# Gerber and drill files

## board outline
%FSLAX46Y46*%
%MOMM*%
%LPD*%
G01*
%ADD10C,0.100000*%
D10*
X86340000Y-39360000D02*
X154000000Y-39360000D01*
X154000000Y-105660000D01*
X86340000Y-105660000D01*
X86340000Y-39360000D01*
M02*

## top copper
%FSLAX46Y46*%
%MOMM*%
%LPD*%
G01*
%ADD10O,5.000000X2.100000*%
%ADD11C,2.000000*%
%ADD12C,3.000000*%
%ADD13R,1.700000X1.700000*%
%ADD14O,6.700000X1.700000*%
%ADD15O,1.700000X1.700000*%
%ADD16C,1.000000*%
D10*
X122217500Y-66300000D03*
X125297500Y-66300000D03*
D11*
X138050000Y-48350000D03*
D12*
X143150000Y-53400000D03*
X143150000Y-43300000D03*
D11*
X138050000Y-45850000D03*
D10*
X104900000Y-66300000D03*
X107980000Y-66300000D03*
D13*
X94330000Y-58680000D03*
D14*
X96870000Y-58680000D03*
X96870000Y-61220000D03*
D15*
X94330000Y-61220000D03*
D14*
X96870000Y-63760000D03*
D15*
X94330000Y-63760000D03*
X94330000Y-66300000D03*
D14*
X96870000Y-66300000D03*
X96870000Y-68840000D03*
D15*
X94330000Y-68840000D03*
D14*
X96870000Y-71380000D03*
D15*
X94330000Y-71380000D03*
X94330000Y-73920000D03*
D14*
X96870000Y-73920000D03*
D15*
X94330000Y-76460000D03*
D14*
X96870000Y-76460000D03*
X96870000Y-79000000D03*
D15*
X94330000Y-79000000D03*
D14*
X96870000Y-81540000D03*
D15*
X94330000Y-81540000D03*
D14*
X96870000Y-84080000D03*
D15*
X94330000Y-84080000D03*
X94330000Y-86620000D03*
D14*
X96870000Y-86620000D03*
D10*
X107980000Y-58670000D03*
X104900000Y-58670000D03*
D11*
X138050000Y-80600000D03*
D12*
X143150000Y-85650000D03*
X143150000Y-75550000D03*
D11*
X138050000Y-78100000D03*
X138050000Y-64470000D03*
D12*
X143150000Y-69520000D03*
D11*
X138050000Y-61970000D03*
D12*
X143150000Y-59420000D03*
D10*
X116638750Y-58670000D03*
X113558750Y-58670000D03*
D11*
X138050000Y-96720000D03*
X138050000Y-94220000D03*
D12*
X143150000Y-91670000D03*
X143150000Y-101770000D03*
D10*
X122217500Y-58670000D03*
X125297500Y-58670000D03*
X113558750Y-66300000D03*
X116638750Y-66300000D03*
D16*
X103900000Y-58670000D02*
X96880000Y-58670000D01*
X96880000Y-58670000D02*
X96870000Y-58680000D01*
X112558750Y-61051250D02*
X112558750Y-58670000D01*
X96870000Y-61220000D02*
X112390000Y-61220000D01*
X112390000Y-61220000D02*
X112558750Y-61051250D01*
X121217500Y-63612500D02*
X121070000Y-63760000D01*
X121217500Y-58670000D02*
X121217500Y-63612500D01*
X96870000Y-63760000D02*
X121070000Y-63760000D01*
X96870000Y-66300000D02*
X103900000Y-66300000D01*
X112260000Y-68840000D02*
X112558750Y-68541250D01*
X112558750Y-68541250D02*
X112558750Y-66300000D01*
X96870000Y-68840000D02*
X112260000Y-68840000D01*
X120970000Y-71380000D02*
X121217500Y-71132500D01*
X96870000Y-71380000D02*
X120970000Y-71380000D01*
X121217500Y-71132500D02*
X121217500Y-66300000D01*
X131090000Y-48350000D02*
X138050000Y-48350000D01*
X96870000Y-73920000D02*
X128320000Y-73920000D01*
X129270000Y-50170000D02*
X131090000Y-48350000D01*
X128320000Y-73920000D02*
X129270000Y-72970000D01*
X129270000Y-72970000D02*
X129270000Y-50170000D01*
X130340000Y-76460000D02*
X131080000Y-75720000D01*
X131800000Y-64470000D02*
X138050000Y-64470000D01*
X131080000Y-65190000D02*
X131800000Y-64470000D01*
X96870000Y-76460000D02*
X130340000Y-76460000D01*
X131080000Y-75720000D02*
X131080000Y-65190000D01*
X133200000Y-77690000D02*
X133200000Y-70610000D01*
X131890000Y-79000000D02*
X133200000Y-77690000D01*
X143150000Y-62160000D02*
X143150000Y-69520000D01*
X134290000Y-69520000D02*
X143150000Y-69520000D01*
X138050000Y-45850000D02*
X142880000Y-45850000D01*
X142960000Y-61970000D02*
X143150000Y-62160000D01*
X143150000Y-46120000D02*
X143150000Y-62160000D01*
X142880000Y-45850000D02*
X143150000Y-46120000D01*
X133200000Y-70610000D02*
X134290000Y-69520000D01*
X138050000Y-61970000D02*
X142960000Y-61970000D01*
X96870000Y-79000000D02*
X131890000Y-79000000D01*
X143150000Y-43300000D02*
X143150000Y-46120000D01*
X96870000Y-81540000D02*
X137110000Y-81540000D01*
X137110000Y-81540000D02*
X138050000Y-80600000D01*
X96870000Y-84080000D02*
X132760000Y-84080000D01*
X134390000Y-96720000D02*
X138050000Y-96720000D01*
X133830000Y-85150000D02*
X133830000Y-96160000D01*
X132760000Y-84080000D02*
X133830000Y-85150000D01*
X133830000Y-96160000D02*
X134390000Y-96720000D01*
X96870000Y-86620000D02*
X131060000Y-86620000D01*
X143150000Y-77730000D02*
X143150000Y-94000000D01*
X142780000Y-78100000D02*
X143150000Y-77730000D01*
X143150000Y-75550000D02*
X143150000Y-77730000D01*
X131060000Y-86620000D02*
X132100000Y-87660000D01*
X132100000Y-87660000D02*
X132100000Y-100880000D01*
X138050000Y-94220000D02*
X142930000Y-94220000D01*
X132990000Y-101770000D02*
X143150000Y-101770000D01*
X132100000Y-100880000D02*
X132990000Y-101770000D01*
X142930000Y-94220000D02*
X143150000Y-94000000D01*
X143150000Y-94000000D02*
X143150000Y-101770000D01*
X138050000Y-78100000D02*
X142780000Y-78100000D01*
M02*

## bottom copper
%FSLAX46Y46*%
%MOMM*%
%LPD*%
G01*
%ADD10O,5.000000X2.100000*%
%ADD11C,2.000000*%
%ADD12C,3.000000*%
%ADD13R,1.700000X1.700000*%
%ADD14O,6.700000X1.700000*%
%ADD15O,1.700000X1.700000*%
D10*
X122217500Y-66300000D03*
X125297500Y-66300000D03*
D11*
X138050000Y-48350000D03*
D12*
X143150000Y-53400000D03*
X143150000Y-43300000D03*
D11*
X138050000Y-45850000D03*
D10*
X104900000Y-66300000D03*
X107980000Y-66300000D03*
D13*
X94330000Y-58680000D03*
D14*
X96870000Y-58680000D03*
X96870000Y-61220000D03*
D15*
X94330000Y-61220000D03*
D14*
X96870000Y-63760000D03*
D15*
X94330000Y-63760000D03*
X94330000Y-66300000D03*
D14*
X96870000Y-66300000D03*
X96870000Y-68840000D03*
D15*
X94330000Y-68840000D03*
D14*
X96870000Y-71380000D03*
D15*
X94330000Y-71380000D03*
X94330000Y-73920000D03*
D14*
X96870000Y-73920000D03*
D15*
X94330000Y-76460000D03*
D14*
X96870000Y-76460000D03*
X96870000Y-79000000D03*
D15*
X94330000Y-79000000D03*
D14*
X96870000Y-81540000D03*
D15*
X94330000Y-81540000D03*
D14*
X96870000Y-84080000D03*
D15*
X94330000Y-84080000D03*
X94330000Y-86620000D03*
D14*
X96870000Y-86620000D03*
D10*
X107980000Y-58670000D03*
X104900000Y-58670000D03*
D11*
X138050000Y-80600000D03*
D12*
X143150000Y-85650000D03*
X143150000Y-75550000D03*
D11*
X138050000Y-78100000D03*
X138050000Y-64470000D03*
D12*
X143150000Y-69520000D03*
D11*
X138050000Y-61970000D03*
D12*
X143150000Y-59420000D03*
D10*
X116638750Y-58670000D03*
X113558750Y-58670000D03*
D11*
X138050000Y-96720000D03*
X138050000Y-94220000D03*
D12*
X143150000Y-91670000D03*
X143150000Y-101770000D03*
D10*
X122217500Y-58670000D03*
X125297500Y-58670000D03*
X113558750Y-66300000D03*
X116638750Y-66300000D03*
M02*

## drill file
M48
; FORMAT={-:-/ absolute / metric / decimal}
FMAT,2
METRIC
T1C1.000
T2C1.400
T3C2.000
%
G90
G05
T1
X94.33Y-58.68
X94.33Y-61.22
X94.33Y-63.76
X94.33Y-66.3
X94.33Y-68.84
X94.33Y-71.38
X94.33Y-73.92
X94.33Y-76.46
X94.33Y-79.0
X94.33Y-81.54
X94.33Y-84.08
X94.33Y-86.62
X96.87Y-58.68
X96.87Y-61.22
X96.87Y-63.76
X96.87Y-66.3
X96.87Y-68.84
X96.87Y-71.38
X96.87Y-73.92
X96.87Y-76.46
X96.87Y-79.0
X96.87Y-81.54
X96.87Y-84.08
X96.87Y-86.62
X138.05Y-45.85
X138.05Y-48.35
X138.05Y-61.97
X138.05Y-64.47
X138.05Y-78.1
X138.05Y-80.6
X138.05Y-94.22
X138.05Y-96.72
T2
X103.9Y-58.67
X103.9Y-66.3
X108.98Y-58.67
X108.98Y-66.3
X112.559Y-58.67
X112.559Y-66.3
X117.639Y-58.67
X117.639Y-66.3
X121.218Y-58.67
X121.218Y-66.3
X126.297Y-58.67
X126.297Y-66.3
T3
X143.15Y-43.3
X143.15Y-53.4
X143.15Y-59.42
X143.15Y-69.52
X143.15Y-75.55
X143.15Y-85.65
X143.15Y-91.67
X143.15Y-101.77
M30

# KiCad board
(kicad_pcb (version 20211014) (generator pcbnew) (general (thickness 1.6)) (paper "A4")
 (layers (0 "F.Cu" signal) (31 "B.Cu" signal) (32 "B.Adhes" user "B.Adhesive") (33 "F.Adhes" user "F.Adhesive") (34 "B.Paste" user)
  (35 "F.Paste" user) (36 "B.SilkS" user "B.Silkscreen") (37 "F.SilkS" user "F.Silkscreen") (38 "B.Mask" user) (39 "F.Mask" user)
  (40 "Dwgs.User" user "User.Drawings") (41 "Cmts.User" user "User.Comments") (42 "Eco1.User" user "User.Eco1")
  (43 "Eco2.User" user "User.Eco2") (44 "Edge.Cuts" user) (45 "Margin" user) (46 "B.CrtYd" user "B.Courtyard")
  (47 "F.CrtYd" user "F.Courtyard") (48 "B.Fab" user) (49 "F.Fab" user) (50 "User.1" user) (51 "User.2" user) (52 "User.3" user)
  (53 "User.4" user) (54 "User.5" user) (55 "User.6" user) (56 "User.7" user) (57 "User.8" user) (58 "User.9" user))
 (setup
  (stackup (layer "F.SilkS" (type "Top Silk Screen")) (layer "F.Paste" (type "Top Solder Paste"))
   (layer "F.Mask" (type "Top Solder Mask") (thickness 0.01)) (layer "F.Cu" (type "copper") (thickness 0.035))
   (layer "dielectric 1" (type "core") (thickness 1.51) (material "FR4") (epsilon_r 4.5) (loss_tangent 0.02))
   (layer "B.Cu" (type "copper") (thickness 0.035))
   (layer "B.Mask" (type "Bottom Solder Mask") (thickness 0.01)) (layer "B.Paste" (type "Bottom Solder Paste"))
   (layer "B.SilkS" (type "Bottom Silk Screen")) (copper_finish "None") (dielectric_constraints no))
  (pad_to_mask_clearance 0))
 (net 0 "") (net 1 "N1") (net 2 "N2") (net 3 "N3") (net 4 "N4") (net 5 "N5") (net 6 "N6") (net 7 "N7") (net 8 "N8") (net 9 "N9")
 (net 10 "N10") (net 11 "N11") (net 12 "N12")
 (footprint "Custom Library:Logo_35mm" (layer "F.Cu") (at 114.7 49.1)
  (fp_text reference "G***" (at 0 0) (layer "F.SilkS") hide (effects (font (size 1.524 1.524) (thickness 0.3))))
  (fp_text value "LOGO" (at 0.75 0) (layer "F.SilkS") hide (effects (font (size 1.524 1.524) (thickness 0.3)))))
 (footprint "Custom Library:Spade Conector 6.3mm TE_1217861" (layer "F.Cu") (at 123.7575 66.3)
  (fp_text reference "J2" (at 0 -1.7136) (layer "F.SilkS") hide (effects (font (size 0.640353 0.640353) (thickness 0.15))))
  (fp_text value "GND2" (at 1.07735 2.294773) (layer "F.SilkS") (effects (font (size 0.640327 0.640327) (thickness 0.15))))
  (pad "1" thru_hole oval (at -2.54 0) (size 5 2.1) (drill 1.4 (offset 1 0)) (layers *.Cu *.Mask) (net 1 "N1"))
  (pad "1" thru_hole oval (at 2.54 0) (size 5 2.1) (drill 1.4 (offset -1 0)) (layers *.Cu *.Mask) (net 1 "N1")))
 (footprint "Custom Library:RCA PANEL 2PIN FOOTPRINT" (layer "F.Cu") (at 140.6 48.35 180)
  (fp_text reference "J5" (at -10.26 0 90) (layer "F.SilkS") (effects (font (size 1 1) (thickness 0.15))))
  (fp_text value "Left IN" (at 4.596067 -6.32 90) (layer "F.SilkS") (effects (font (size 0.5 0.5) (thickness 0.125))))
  (pad "1" thru_hole circle (at 2.55 0 180) (size 2 2) (drill 1) (layers *.Cu *.Mask) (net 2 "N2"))
  (pad "2" thru_hole circle (at -2.55 -5.05 180) (size 3 3) (drill 2) (layers *.Cu *.Mask) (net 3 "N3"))
  (pad "2" thru_hole circle (at -2.55 5.05 180) (size 3 3) (drill 2) (layers *.Cu *.Mask) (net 3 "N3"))
  (pad "2" thru_hole circle (at 2.55 2.5 180) (size 2 2) (drill 1) (layers *.Cu *.Mask) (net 3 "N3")))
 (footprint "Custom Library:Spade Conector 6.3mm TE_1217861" (layer "F.Cu") (at 106.44 66.3)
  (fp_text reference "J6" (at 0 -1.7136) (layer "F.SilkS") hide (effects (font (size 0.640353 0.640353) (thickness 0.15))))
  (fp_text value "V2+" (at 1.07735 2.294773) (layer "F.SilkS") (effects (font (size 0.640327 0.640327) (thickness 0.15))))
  (pad "1" thru_hole oval (at -2.54 0) (size 5 2.1) (drill 1.4 (offset 1 0)) (layers *.Cu *.Mask) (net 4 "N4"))
  (pad "1" thru_hole oval (at 2.54 0) (size 5 2.1) (drill 1.4 (offset -1 0)) (layers *.Cu *.Mask) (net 4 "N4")))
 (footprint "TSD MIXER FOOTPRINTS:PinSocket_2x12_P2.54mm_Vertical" (layer "F.Cu") (at 94.33 58.68)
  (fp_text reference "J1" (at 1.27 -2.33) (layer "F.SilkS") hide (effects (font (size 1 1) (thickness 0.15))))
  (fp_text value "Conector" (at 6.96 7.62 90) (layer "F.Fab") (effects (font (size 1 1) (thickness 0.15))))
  (pad "1" thru_hole rect (at 0 0) (size 1.7 1.7) (drill 1) (layers *.Cu *.Mask) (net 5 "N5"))
  (pad "1" thru_hole oval (at 2.54 0) (size 6.7 1.7) (drill 1) (layers *.Cu *.Mask) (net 5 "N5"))
  (pad "2" thru_hole oval (at 2.54 2.54) (size 6.7 1.7) (drill 1) (layers *.Cu *.Mask) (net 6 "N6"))
  (pad "2" thru_hole oval (at 0 2.54) (size 1.7 1.7) (drill 1) (layers *.Cu *.Mask) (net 6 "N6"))
  (pad "3" thru_hole oval (at 2.54 5.08) (size 6.7 1.7) (drill 1) (layers *.Cu *.Mask) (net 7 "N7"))
  (pad "3" thru_hole oval (at 0 5.08) (size 1.7 1.7) (drill 1) (layers *.Cu *.Mask) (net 7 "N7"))
  (pad "4" thru_hole oval (at 0 7.62) (size 1.7 1.7) (drill 1) (layers *.Cu *.Mask) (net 4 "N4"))
  (pad "4" thru_hole oval (at 2.54 7.62) (size 6.7 1.7) (drill 1) (layers *.Cu *.Mask) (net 4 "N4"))
  (pad "5" thru_hole oval (at 2.54 10.16) (size 6.7 1.7) (drill 1) (layers *.Cu *.Mask) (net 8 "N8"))
  (pad "5" thru_hole oval (at 0 10.16) (size 1.7 1.7) (drill 1) (layers *.Cu *.Mask) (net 8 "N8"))
  (pad "6" thru_hole oval (at 2.54 12.7) (size 6.7 1.7) (drill 1) (layers *.Cu *.Mask) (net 1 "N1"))
  (pad "6" thru_hole oval (at 0 12.7) (size 1.7 1.7) (drill 1) (layers *.Cu *.Mask) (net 1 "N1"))
  (pad "7" thru_hole oval (at 0 15.24) (size 1.7 1.7) (drill 1) (layers *.Cu *.Mask) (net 2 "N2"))
  (pad "7" thru_hole oval (at 2.54 15.24) (size 6.7 1.7) (drill 1) (layers *.Cu *.Mask) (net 2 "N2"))
  (pad "8" thru_hole oval (at 0 17.78) (size 1.7 1.7) (drill 1) (layers *.Cu *.Mask) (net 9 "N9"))
  (pad "8" thru_hole oval (at 2.54 17.78) (size 6.7 1.7) (drill 1) (layers *.Cu *.Mask) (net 9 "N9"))
  (pad "9" thru_hole oval (at 2.54 20.32) (size 6.7 1.7) (drill 1) (layers *.Cu *.Mask) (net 3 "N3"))
  (pad "9" thru_hole oval (at 0 20.32) (size 1.7 1.7) (drill 1) (layers *.Cu *.Mask) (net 3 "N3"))
  (pad "10" thru_hole oval (at 2.54 22.86) (size 6.7 1.7) (drill 1) (layers *.Cu *.Mask) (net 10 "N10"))
  (pad "10" thru_hole oval (at 0 22.86) (size 1.7 1.7) (drill 1) (layers *.Cu *.Mask) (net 10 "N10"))
  (pad "11" thru_hole oval (at 2.54 25.4) (size 6.7 1.7) (drill 1) (layers *.Cu *.Mask) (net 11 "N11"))
  (pad "11" thru_hole oval (at 0 25.4) (size 1.7 1.7) (drill 1) (layers *.Cu *.Mask) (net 11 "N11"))
  (pad "12" thru_hole oval (at 0 27.94) (size 1.7 1.7) (drill 1) (layers *.Cu *.Mask) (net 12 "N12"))
  (pad "12" thru_hole oval (at 2.54 27.94) (size 6.7 1.7) (drill 1) (layers *.Cu *.Mask) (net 12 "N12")))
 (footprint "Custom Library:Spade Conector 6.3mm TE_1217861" (layer "F.Cu") (at 106.44 58.67)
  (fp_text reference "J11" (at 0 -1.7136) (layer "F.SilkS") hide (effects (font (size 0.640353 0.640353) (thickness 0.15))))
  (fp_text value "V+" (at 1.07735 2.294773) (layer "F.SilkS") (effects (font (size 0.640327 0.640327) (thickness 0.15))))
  (pad "1" thru_hole oval (at 2.54 0) (size 5 2.1) (drill 1.4 (offset -1 0)) (layers *.Cu *.Mask) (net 5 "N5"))
  (pad "1" thru_hole oval (at -2.54 0) (size 5 2.1) (drill 1.4 (offset 1 0)) (layers *.Cu *.Mask) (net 5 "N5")))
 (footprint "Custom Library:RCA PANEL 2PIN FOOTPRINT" (layer "F.Cu") (at 140.6 80.6 180)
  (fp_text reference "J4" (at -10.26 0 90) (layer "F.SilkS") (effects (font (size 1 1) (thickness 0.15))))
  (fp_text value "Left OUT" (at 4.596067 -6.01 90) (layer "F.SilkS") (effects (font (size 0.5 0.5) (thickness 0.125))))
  (pad "1" thru_hole circle (at 2.55 0 180) (size 2 2) (drill 1) (layers *.Cu *.Mask) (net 10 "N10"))
  (pad "2" thru_hole circle (at -2.55 -5.05 180) (size 3 3) (drill 2) (layers *.Cu *.Mask) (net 12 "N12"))
  (pad "2" thru_hole circle (at -2.55 5.05 180) (size 3 3) (drill 2) (layers *.Cu *.Mask) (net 12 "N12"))
  (pad "2" thru_hole circle (at 2.55 2.5 180) (size 2 2) (drill 1) (layers *.Cu *.Mask) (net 12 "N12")))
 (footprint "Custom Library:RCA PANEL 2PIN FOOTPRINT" (layer "F.Cu") (at 140.6 64.47 180)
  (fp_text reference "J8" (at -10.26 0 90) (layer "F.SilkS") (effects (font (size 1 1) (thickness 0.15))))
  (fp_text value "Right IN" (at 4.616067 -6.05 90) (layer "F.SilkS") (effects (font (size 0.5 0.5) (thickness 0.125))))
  (pad "1" thru_hole circle (at 2.55 0 180) (size 2 2) (drill 1) (layers *.Cu *.Mask) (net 9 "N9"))
  (pad "2" thru_hole circle (at -2.55 -5.05 180) (size 3 3) (drill 2) (layers *.Cu *.Mask) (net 3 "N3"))
  (pad "2" thru_hole circle (at 2.55 2.5 180) (size 2 2) (drill 1) (layers *.Cu *.Mask) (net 3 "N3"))
  (pad "2" thru_hole circle (at -2.55 5.05 180) (size 3 3) (drill 2) (layers *.Cu *.Mask) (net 3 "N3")))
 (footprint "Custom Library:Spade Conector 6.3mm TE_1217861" (layer "F.Cu") (at 115.09875 58.67)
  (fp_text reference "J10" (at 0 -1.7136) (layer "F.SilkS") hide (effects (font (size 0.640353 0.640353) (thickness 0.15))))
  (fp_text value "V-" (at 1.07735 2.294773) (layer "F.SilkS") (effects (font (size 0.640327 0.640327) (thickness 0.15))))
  (pad "1" thru_hole oval (at 2.54 0) (size 5 2.1) (drill 1.4 (offset -1 0)) (layers *.Cu *.Mask) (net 6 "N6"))
  (pad "1" thru_hole oval (at -2.54 0) (size 5 2.1) (drill 1.4 (offset 1 0)) (layers *.Cu *.Mask) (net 6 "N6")))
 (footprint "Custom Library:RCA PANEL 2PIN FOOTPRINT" (layer "F.Cu") (at 140.6 96.72 180)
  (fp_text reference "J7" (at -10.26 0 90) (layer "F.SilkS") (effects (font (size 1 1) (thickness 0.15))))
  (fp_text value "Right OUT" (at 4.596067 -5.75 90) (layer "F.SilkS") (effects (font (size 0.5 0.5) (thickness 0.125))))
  (pad "1" thru_hole circle (at 2.55 0 180) (size 2 2) (drill 1) (layers *.Cu *.Mask) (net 11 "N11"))
  (pad "2" thru_hole circle (at 2.55 2.5 180) (size 2 2) (drill 1) (layers *.Cu *.Mask) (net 12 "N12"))
  (pad "2" thru_hole circle (at -2.55 5.05 180) (size 3 3) (drill 2) (layers *.Cu *.Mask) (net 12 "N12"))
  (pad "2" thru_hole circle (at -2.55 -5.05 180) (size 3 3) (drill 2) (layers *.Cu *.Mask) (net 12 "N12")))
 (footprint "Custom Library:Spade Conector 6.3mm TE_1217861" (layer "F.Cu") (at 123.7575 58.67)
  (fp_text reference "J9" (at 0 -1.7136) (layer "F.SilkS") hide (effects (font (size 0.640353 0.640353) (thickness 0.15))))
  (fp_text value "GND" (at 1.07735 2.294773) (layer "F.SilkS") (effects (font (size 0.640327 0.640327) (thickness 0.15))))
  (pad "1" thru_hole oval (at -2.54 0) (size 5 2.1) (drill 1.4 (offset 1 0)) (layers *.Cu *.Mask) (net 7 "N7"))
  (pad "1" thru_hole oval (at 2.54 0) (size 5 2.1) (drill 1.4 (offset -1 0)) (layers *.Cu *.Mask) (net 7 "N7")))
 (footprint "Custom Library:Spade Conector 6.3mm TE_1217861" (layer "F.Cu") (at 115.09875 66.3)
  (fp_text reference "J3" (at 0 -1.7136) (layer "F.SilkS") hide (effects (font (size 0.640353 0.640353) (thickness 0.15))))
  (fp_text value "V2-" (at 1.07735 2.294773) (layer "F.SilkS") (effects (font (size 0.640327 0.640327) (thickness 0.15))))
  (pad "1" thru_hole oval (at -2.54 0) (size 5 2.1) (drill 1.4 (offset 1 0)) (layers *.Cu *.Mask) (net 8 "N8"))
  (pad "1" thru_hole oval (at 2.54 0) (size 5 2.1) (drill 1.4 (offset -1 0)) (layers *.Cu *.Mask) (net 8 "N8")))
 (gr_rect (start 154 39.36) (end 86.34 105.66) (layer "Edge.Cuts") (width 0.1) (fill none))
 (segment (start 103.9 58.67) (end 96.88 58.67) (width 1) (layer "F.Cu") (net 5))
 (segment (start 96.88 58.67) (end 96.87 58.68) (width 1) (layer "F.Cu") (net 5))
 (segment (start 112.55875 61.05125) (end 112.55875 58.67) (width 1) (layer "F.Cu") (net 6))
 (segment (start 96.87 61.22) (end 112.39 61.22) (width 1) (layer "F.Cu") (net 6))
 (segment (start 112.39 61.22) (end 112.55875 61.05125) (width 1) (layer "F.Cu") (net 6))
 (segment (start 121.2175 63.6125) (end 121.07 63.76) (width 1) (layer "F.Cu") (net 7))
 (segment (start 121.2175 58.67) (end 121.2175 63.6125) (width 1) (layer "F.Cu") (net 7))
 (segment (start 96.87 63.76) (end 121.07 63.76) (width 1) (layer "F.Cu") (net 7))
 (segment (start 96.87 66.3) (end 103.9 66.3) (width 1) (layer "F.Cu") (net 4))
 (segment (start 112.26 68.84) (end 112.55875 68.54125) (width 1) (layer "F.Cu") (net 8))
 (segment (start 112.55875 68.54125) (end 112.55875 66.3) (width 1) (layer "F.Cu") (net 8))
 (segment (start 96.87 68.84) (end 112.26 68.84) (width 1) (layer "F.Cu") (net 8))
 (segment (start 120.97 71.38) (end 121.2175 71.1325) (width 1) (layer "F.Cu") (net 1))
 (segment (start 96.87 71.38) (end 120.97 71.38) (width 1) (layer "F.Cu") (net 1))
 (segment (start 121.2175 71.1325) (end 121.2175 66.3) (width 1) (layer "F.Cu") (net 1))
 (segment (start 131.09 48.35) (end 138.05 48.35) (width 1) (layer "F.Cu") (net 2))
 (segment (start 96.87 73.92) (end 128.32 73.92) (width 1) (layer "F.Cu") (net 2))
 (segment (start 129.27 50.17) (end 131.09 48.35) (width 1) (layer "F.Cu") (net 2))
 (segment (start 128.32 73.92) (end 129.27 72.97) (width 1) (layer "F.Cu") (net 2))
 (segment (start 129.27 72.97) (end 129.27 50.17) (width 1) (layer "F.Cu") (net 2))
 (segment (start 130.34 76.46) (end 131.08 75.72) (width 1) (layer "F.Cu") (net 9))
 (segment (start 131.8 64.47) (end 138.05 64.47) (width 1) (layer "F.Cu") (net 9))
 (segment (start 131.08 65.19) (end 131.8 64.47) (width 1) (layer "F.Cu") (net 9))
 (segment (start 96.87 76.46) (end 130.34 76.46) (width 1) (layer "F.Cu") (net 9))
 (segment (start 131.08 75.72) (end 131.08 65.19) (width 1) (layer "F.Cu") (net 9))
 (segment (start 133.2 77.69) (end 133.2 70.61) (width 1) (layer "F.Cu") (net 3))
 (segment (start 131.89 79) (end 133.2 77.69) (width 1) (layer "F.Cu") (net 3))
 (segment (start 143.15 62.16) (end 143.15 69.52) (width 1) (layer "F.Cu") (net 3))
 (segment (start 134.29 69.52) (end 143.15 69.52) (width 1) (layer "F.Cu") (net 3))
 (segment (start 138.05 45.85) (end 142.88 45.85) (width 1) (layer "F.Cu") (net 3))
 (segment (start 142.96 61.97) (end 143.15 62.16) (width 1) (layer "F.Cu") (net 3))
 (segment (start 143.15 46.12) (end 143.15 62.16) (width 1) (layer "F.Cu") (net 3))
 (segment (start 142.88 45.85) (end 143.15 46.12) (width 1) (layer "F.Cu") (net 3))
 (segment (start 133.2 70.61) (end 134.29 69.52) (width 1) (layer "F.Cu") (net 3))
 (segment (start 138.05 61.97) (end 142.96 61.97) (width 1) (layer "F.Cu") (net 3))
 (segment (start 96.87 79) (end 131.89 79) (width 1) (layer "F.Cu") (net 3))
 (segment (start 143.15 43.3) (end 143.15 46.12) (width 1) (layer "F.Cu") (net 3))
 (segment (start 96.87 81.54) (end 137.11 81.54) (width 1) (layer "F.Cu") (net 10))
 (segment (start 137.11 81.54) (end 138.05 80.6) (width 1) (layer "F.Cu") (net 10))
 (segment (start 96.87 84.08) (end 132.76 84.08) (width 1) (layer "F.Cu") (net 11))
 (segment (start 134.39 96.72) (end 138.05 96.72) (width 1) (layer "F.Cu") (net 11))
 (segment (start 133.83 85.15) (end 133.83 96.16) (width 1) (layer "F.Cu") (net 11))
 (segment (start 132.76 84.08) (end 133.83 85.15) (width 1) (layer "F.Cu") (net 11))
 (segment (start 133.83 96.16) (end 134.39 96.72) (width 1) (layer "F.Cu") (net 11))
 (segment (start 96.87 86.62) (end 131.06 86.62) (width 1) (layer "F.Cu") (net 12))
 (segment (start 143.15 77.73) (end 143.15 94) (width 1) (layer "F.Cu") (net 12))
 (segment (start 142.78 78.1) (end 143.15 77.73) (width 1) (layer "F.Cu") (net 12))
 (segment (start 143.15 75.55) (end 143.15 77.73) (width 1) (layer "F.Cu") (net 12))
 (segment (start 131.06 86.62) (end 132.1 87.66) (width 1) (layer "F.Cu") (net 12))
 (segment (start 132.1 87.66) (end 132.1 100.88) (width 1) (layer "F.Cu") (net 12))
 (segment (start 138.05 94.22) (end 142.93 94.22) (width 1) (layer "F.Cu") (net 12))
 (segment (start 132.99 101.77) (end 143.15 101.77) (width 1) (layer "F.Cu") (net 12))
 (segment (start 132.1 100.88) (end 132.99 101.77) (width 1) (layer "F.Cu") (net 12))
 (segment (start 142.93 94.22) (end 143.15 94) (width 1) (layer "F.Cu") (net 12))
 (segment (start 143.15 94) (end 143.15 101.77) (width 1) (layer "F.Cu") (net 12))
 (segment (start 138.05 78.1) (end 142.78 78.1) (width 1) (layer "F.Cu") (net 12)))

